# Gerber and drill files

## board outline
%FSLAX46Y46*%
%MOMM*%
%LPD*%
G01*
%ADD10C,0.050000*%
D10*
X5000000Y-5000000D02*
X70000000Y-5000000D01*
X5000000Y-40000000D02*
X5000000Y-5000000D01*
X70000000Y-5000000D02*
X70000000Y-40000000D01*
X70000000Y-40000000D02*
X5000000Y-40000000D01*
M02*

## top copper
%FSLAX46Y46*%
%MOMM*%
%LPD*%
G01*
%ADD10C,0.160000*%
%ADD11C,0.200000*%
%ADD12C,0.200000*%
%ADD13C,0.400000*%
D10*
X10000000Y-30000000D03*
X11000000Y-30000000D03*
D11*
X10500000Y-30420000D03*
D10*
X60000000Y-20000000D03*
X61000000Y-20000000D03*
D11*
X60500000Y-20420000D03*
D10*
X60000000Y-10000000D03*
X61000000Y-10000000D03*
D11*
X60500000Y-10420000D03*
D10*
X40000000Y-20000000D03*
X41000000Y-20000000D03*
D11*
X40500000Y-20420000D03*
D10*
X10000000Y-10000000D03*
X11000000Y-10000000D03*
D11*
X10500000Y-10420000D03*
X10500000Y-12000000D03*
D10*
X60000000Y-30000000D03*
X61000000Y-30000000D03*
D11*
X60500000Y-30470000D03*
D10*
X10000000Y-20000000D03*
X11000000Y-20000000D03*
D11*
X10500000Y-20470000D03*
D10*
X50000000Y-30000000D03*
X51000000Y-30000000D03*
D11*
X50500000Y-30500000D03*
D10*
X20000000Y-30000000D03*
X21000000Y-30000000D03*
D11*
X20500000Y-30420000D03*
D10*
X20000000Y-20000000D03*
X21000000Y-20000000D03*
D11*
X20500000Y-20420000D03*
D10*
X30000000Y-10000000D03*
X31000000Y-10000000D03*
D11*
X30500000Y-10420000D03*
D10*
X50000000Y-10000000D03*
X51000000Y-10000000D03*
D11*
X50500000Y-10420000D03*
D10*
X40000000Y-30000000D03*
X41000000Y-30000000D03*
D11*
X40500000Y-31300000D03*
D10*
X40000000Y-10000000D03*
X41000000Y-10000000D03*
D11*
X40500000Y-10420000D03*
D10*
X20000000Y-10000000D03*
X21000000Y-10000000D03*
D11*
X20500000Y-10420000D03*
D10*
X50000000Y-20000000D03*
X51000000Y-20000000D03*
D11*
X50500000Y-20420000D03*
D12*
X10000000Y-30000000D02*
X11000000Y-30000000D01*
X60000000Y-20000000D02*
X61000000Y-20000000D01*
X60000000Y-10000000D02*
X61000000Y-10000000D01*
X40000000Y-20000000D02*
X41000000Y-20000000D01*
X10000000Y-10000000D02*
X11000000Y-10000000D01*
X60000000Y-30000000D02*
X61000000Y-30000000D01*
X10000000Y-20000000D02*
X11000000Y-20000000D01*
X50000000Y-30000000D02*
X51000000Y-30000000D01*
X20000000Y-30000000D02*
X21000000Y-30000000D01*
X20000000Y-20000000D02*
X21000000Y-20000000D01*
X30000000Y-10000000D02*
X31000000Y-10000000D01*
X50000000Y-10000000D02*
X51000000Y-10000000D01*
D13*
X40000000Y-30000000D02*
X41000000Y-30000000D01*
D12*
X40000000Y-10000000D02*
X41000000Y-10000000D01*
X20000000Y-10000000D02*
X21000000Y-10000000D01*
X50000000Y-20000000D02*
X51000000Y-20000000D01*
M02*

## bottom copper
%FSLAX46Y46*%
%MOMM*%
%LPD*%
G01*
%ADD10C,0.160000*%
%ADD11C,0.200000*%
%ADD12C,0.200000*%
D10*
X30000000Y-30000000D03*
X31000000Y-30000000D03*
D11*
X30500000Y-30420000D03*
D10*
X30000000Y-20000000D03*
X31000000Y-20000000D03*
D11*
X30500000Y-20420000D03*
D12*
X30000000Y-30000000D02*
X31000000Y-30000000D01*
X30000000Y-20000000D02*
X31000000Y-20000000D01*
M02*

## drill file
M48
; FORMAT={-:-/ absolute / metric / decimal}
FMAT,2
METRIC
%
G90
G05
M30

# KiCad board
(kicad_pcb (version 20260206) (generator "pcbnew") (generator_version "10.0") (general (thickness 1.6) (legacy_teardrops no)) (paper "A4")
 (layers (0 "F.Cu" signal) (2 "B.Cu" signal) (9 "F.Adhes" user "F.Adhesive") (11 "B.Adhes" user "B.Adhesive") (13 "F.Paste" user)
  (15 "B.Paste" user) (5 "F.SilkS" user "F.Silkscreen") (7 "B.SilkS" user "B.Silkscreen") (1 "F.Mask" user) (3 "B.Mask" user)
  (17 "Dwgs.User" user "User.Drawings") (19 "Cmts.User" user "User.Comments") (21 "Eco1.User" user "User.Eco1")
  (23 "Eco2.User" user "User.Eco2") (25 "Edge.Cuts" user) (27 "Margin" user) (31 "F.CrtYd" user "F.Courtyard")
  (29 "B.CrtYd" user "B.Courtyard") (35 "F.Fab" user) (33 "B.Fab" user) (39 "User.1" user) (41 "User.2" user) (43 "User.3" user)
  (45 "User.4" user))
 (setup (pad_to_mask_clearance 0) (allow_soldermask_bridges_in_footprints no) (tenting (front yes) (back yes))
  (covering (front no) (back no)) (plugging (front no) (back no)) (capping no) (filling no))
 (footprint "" (layer "F.Cu") (at 10 30)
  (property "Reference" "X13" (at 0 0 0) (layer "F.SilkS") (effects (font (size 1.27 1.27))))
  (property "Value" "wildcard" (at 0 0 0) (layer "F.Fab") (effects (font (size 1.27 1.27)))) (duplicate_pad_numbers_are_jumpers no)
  (pad "1" smd circle (at 0 0) (size 0.16 0.16) (layers "F.Cu") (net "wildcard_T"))
  (pad "2" smd circle (at 1 0) (size 0.16 0.16) (layers "F.Cu") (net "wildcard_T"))
  (pad "3" smd circle (at 0.5 0.42) (size 0.2 0.2) (layers "F.Cu") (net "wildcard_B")))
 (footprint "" (layer "F.Cu") (at 60 20)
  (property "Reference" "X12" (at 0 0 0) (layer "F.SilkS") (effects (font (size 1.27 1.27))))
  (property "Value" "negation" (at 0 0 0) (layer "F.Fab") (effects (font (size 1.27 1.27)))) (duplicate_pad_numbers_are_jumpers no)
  (pad "1" smd circle (at 0 0) (size 0.16 0.16) (layers "F.Cu") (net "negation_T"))
  (pad "2" smd circle (at 1 0) (size 0.16 0.16) (layers "F.Cu") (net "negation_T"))
  (pad "3" smd circle (at 0.5 0.42) (size 0.2 0.2) (layers "F.Cu") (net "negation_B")))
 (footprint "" (layer "F.Cu") (at 60 10)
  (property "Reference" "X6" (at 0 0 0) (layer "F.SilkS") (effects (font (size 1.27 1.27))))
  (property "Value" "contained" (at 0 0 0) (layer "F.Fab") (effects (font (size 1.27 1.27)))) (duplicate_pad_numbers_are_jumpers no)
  (pad "1" smd circle (at 0 0) (size 0.16 0.16) (layers "F.Cu") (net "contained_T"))
  (pad "2" smd circle (at 1 0) (size 0.16 0.16) (layers "F.Cu") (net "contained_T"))
  (pad "3" smd circle (at 0.5 0.42) (size 0.2 0.2) (layers "F.Cu") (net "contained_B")))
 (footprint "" (layer "F.Cu") (at 40 20)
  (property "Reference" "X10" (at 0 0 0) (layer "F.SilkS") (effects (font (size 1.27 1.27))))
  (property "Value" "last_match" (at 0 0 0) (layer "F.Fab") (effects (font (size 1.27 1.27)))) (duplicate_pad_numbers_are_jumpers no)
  (pad "1" smd circle (at 0 0) (size 0.16 0.16) (layers "F.Cu") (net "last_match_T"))
  (pad "2" smd circle (at 1 0) (size 0.16 0.16) (layers "F.Cu") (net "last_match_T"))
  (pad "3" smd circle (at 0.5 0.42) (size 0.2 0.2) (layers "F.Cu") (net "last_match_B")))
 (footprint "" (layer "F.Cu") (at 10 10)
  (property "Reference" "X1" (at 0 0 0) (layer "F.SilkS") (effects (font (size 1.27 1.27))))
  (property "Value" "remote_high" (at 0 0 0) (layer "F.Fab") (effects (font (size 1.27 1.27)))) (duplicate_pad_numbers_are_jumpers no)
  (pad "1" smd circle (at 0 0) (size 0.16 0.16) (layers "F.Cu") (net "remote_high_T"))
  (pad "2" smd circle (at 1 0) (size 0.16 0.16) (layers "F.Cu") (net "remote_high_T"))
  (pad "3" smd circle (at 0.5 0.42) (size 0.2 0.2) (layers "F.Cu") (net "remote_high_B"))
  (pad "4" smd circle (at 0.5 2) (size 0.2 0.2) (layers "F.Cu") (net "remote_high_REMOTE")))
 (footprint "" (layer "F.Cu") (at 60 30)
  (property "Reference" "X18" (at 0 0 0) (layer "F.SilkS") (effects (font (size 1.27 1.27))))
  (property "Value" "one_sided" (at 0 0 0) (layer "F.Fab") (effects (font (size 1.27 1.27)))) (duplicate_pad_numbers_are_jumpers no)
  (pad "1" smd circle (at 0 0) (size 0.16 0.16) (layers "F.Cu") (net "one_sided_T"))
  (pad "2" smd circle (at 1 0) (size 0.16 0.16) (layers "F.Cu") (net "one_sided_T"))
  (pad "3" smd circle (at 0.5 0.47) (size 0.2 0.2) (layers "F.Cu") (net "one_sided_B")))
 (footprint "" (layer "F.Cu") (at 10 20)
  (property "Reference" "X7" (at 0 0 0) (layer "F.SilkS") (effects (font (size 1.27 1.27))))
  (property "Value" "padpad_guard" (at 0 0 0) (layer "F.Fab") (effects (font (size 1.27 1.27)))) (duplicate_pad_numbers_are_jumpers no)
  (pad "1" smd circle (at 0 0) (size 0.16 0.16) (layers "F.Cu") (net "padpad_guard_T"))
  (pad "2" smd circle (at 1 0) (size 0.16 0.16) (layers "F.Cu") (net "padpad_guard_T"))
  (pad "3" smd circle (at 0.5 0.47) (size 0.2 0.2) (layers "F.Cu") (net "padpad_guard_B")))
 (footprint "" (layer "F.Cu") (at 50 30)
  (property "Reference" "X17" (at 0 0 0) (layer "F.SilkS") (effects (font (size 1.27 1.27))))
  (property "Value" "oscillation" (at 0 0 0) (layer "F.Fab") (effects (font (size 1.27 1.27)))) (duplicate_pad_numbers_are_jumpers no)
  (pad "1" smd circle (at 0 0) (size 0.16 0.16) (layers "F.Cu") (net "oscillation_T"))
  (pad "2" smd circle (at 1 0) (size 0.16 0.16) (layers "F.Cu") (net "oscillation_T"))
  (pad "3" smd circle (at 0.5 0.5) (size 0.2 0.2) (layers "F.Cu") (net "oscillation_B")))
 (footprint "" (layer "F.Cu") (at 20 30)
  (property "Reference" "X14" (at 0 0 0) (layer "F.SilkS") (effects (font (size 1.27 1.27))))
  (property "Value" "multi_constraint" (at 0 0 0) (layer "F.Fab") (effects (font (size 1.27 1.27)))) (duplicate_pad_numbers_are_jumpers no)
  (pad "1" smd circle (at 0 0) (size 0.16 0.16) (layers "F.Cu") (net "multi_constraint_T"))
  (pad "2" smd circle (at 1 0) (size 0.16 0.16) (layers "F.Cu") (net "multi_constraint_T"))
  (pad "3" smd circle (at 0.5 0.42) (size 0.2 0.2) (layers "F.Cu") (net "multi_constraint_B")))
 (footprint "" (layer "F.Cu") (at 30 30)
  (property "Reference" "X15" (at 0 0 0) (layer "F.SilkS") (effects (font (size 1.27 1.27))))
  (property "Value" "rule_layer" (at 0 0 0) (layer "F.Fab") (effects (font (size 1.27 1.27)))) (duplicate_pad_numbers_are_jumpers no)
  (pad "1" smd circle (at 0 0) (size 0.16 0.16) (layers "B.Cu") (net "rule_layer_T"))
  (pad "2" smd circle (at 1 0) (size 0.16 0.16) (layers "B.Cu") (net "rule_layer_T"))
  (pad "3" smd circle (at 0.5 0.42) (size 0.2 0.2) (layers "B.Cu") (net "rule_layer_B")))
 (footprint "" (layer "F.Cu") (at 20 20)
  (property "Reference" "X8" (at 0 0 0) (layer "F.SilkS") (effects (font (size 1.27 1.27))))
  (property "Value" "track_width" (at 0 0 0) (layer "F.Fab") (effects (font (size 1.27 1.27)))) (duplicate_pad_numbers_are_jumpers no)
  (pad "1" smd circle (at 0 0) (size 0.16 0.16) (layers "F.Cu") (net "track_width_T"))
  (pad "2" smd circle (at 1 0) (size 0.16 0.16) (layers "F.Cu") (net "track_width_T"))
  (pad "3" smd circle (at 0.5 0.42) (size 0.2 0.2) (layers "F.Cu") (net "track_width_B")))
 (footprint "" (layer "F.Cu") (at 30 10)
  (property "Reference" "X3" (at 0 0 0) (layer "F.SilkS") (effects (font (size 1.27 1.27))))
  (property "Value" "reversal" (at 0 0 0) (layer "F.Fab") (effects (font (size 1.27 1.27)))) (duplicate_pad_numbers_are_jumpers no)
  (pad "1" smd circle (at 0 0) (size 0.16 0.16) (layers "F.Cu") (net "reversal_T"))
  (pad "2" smd circle (at 1 0) (size 0.16 0.16) (layers "F.Cu") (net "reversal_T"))
  (pad "3" smd circle (at 0.5 0.42) (size 0.2 0.2) (layers "F.Cu") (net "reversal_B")))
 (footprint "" (layer "F.Cu") (at 50 10)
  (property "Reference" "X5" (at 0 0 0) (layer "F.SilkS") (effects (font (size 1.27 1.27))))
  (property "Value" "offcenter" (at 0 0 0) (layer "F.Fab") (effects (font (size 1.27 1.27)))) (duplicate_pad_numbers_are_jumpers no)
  (pad "1" smd circle (at 0 0) (size 0.16 0.16) (layers "F.Cu") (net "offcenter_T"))
  (pad "2" smd circle (at 1 0) (size 0.16 0.16) (layers "F.Cu") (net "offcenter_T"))
  (pad "3" smd circle (at 0.5 0.42) (size 0.2 0.2) (layers "F.Cu") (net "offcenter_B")))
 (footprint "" (layer "F.Cu") (at 40 30)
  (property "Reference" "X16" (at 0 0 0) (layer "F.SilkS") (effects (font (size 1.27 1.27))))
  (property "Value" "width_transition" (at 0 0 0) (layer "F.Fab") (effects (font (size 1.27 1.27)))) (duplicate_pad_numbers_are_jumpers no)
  (pad "1" smd circle (at 0 0) (size 0.16 0.16) (layers "F.Cu") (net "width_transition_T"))
  (pad "2" smd circle (at 1 0) (size 0.16 0.16) (layers "F.Cu") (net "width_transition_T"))
  (pad "3" smd circle (at 0.5 1.3) (size 0.2 0.2) (layers "F.Cu") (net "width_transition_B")))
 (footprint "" (layer "F.Cu") (at 30 20)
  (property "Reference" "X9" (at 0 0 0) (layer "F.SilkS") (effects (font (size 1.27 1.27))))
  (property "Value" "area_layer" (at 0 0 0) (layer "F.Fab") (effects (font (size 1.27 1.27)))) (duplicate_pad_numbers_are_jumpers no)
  (pad "1" smd circle (at 0 0) (size 0.16 0.16) (layers "B.Cu") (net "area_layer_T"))
  (pad "2" smd circle (at 1 0) (size 0.16 0.16) (layers "B.Cu") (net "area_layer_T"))
  (pad "3" smd circle (at 0.5 0.42) (size 0.2 0.2) (layers "B.Cu") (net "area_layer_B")))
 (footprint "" (layer "F.Cu") (at 40 10)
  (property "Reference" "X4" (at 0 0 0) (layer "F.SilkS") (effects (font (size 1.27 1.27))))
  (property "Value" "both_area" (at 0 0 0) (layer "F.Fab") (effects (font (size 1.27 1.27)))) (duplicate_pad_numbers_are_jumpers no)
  (pad "1" smd circle (at 0 0) (size 0.16 0.16) (layers "F.Cu") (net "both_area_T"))
  (pad "2" smd circle (at 1 0) (size 0.16 0.16) (layers "F.Cu") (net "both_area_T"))
  (pad "3" smd circle (at 0.5 0.42) (size 0.2 0.2) (layers "F.Cu") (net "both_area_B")))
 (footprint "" (layer "F.Cu") (at 20 10)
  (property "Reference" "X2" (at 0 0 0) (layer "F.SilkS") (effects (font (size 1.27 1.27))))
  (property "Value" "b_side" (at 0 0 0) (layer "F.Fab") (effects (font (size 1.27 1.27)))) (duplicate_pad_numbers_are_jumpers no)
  (pad "1" smd circle (at 0 0) (size 0.16 0.16) (layers "F.Cu") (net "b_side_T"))
  (pad "2" smd circle (at 1 0) (size 0.16 0.16) (layers "F.Cu") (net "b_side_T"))
  (pad "3" smd circle (at 0.5 0.42) (size 0.2 0.2) (layers "F.Cu") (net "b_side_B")))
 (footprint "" (layer "F.Cu") (at 50 20)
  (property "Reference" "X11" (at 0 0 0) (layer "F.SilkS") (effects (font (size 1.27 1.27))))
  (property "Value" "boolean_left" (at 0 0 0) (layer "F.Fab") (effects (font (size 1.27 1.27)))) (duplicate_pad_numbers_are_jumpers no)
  (pad "1" smd circle (at 0 0) (size 0.16 0.16) (layers "F.Cu") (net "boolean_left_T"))
  (pad "2" smd circle (at 1 0) (size 0.16 0.16) (layers "F.Cu") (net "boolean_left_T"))
  (pad "3" smd circle (at 0.5 0.42) (size 0.2 0.2) (layers "F.Cu") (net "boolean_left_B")))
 (gr_line (start 5 5) (end 70 5) (stroke (width 0.05) (type default)) (layer "Edge.Cuts"))
 (gr_line (start 5 40) (end 5 5) (stroke (width 0.05) (type default)) (layer "Edge.Cuts"))
 (gr_line (start 70 5) (end 70 40) (stroke (width 0.05) (type default)) (layer "Edge.Cuts"))
 (gr_line (start 70 40) (end 5 40) (stroke (width 0.05) (type default)) (layer "Edge.Cuts"))
 (segment (start 10 30) (end 11 30) (width 0.2) (layer "F.Cu") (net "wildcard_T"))
 (segment (start 60 20) (end 61 20) (width 0.2) (layer "F.Cu") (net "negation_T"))
 (segment (start 60 10) (end 61 10) (width 0.2) (layer "F.Cu") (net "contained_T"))
 (segment (start 40 20) (end 41 20) (width 0.2) (layer "F.Cu") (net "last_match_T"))
 (segment (start 10 10) (end 11 10) (width 0.2) (layer "F.Cu") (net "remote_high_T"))
 (segment (start 60 30) (end 61 30) (width 0.2) (layer "F.Cu") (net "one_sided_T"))
 (segment (start 10 20) (end 11 20) (width 0.2) (layer "F.Cu") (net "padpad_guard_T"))
 (segment (start 50 30) (end 51 30) (width 0.2) (layer "F.Cu") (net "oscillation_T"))
 (segment (start 20 30) (end 21 30) (width 0.2) (layer "F.Cu") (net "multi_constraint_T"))
 (segment (start 30 30) (end 31 30) (width 0.2) (layer "B.Cu") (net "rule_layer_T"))
 (segment (start 20 20) (end 21 20) (width 0.2) (layer "F.Cu") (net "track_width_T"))
 (segment (start 30 10) (end 31 10) (width 0.2) (layer "F.Cu") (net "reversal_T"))
 (segment (start 50 10) (end 51 10) (width 0.2) (layer "F.Cu") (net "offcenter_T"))
 (segment (start 40 30) (end 41 30) (width 0.4) (layer "F.Cu") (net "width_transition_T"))
 (segment (start 30 20) (end 31 20) (width 0.2) (layer "B.Cu") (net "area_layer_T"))
 (segment (start 40 10) (end 41 10) (width 0.2) (layer "F.Cu") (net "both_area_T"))
 (segment (start 20 10) (end 21 10) (width 0.2) (layer "F.Cu") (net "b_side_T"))
 (segment (start 50 20) (end 51 20) (width 0.2) (layer "F.Cu") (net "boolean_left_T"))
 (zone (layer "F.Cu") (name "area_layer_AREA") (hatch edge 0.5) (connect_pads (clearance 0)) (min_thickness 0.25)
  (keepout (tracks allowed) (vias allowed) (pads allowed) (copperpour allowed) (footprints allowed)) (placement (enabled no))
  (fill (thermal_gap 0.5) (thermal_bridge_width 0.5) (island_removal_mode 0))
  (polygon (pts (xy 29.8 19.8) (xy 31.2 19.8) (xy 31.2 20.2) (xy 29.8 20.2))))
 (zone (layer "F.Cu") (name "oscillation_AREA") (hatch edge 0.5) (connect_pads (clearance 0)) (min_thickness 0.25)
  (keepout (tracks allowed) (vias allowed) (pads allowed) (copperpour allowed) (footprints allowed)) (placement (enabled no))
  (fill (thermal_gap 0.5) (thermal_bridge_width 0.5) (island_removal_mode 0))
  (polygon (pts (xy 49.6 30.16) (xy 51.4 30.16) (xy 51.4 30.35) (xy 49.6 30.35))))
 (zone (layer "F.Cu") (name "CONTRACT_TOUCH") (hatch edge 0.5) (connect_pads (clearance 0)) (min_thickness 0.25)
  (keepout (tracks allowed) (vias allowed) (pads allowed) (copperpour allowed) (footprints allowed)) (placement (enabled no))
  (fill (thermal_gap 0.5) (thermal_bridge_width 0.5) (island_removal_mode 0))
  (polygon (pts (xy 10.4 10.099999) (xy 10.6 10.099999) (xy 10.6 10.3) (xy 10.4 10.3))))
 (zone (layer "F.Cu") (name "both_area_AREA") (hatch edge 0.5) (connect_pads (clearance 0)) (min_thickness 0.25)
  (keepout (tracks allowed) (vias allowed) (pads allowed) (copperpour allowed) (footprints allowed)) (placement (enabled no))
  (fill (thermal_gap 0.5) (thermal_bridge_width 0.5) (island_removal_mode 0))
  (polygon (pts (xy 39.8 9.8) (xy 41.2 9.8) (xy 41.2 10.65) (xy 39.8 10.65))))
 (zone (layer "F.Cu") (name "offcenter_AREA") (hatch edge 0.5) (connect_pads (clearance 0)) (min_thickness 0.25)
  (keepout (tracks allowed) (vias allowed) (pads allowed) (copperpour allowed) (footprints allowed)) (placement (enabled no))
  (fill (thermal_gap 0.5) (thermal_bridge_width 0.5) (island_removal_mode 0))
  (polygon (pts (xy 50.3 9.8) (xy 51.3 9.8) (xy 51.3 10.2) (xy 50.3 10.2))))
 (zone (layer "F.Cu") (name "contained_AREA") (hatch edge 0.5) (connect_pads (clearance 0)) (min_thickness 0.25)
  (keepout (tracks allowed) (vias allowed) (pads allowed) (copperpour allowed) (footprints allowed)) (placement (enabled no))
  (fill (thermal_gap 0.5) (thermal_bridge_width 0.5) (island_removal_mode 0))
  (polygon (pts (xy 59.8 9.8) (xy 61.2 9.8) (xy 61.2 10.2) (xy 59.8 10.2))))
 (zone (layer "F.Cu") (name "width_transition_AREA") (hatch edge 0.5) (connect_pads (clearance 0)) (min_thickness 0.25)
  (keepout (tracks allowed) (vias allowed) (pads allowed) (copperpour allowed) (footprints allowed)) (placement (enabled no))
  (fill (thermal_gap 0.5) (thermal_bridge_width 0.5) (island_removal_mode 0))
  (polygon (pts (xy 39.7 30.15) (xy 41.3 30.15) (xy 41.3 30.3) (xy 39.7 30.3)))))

